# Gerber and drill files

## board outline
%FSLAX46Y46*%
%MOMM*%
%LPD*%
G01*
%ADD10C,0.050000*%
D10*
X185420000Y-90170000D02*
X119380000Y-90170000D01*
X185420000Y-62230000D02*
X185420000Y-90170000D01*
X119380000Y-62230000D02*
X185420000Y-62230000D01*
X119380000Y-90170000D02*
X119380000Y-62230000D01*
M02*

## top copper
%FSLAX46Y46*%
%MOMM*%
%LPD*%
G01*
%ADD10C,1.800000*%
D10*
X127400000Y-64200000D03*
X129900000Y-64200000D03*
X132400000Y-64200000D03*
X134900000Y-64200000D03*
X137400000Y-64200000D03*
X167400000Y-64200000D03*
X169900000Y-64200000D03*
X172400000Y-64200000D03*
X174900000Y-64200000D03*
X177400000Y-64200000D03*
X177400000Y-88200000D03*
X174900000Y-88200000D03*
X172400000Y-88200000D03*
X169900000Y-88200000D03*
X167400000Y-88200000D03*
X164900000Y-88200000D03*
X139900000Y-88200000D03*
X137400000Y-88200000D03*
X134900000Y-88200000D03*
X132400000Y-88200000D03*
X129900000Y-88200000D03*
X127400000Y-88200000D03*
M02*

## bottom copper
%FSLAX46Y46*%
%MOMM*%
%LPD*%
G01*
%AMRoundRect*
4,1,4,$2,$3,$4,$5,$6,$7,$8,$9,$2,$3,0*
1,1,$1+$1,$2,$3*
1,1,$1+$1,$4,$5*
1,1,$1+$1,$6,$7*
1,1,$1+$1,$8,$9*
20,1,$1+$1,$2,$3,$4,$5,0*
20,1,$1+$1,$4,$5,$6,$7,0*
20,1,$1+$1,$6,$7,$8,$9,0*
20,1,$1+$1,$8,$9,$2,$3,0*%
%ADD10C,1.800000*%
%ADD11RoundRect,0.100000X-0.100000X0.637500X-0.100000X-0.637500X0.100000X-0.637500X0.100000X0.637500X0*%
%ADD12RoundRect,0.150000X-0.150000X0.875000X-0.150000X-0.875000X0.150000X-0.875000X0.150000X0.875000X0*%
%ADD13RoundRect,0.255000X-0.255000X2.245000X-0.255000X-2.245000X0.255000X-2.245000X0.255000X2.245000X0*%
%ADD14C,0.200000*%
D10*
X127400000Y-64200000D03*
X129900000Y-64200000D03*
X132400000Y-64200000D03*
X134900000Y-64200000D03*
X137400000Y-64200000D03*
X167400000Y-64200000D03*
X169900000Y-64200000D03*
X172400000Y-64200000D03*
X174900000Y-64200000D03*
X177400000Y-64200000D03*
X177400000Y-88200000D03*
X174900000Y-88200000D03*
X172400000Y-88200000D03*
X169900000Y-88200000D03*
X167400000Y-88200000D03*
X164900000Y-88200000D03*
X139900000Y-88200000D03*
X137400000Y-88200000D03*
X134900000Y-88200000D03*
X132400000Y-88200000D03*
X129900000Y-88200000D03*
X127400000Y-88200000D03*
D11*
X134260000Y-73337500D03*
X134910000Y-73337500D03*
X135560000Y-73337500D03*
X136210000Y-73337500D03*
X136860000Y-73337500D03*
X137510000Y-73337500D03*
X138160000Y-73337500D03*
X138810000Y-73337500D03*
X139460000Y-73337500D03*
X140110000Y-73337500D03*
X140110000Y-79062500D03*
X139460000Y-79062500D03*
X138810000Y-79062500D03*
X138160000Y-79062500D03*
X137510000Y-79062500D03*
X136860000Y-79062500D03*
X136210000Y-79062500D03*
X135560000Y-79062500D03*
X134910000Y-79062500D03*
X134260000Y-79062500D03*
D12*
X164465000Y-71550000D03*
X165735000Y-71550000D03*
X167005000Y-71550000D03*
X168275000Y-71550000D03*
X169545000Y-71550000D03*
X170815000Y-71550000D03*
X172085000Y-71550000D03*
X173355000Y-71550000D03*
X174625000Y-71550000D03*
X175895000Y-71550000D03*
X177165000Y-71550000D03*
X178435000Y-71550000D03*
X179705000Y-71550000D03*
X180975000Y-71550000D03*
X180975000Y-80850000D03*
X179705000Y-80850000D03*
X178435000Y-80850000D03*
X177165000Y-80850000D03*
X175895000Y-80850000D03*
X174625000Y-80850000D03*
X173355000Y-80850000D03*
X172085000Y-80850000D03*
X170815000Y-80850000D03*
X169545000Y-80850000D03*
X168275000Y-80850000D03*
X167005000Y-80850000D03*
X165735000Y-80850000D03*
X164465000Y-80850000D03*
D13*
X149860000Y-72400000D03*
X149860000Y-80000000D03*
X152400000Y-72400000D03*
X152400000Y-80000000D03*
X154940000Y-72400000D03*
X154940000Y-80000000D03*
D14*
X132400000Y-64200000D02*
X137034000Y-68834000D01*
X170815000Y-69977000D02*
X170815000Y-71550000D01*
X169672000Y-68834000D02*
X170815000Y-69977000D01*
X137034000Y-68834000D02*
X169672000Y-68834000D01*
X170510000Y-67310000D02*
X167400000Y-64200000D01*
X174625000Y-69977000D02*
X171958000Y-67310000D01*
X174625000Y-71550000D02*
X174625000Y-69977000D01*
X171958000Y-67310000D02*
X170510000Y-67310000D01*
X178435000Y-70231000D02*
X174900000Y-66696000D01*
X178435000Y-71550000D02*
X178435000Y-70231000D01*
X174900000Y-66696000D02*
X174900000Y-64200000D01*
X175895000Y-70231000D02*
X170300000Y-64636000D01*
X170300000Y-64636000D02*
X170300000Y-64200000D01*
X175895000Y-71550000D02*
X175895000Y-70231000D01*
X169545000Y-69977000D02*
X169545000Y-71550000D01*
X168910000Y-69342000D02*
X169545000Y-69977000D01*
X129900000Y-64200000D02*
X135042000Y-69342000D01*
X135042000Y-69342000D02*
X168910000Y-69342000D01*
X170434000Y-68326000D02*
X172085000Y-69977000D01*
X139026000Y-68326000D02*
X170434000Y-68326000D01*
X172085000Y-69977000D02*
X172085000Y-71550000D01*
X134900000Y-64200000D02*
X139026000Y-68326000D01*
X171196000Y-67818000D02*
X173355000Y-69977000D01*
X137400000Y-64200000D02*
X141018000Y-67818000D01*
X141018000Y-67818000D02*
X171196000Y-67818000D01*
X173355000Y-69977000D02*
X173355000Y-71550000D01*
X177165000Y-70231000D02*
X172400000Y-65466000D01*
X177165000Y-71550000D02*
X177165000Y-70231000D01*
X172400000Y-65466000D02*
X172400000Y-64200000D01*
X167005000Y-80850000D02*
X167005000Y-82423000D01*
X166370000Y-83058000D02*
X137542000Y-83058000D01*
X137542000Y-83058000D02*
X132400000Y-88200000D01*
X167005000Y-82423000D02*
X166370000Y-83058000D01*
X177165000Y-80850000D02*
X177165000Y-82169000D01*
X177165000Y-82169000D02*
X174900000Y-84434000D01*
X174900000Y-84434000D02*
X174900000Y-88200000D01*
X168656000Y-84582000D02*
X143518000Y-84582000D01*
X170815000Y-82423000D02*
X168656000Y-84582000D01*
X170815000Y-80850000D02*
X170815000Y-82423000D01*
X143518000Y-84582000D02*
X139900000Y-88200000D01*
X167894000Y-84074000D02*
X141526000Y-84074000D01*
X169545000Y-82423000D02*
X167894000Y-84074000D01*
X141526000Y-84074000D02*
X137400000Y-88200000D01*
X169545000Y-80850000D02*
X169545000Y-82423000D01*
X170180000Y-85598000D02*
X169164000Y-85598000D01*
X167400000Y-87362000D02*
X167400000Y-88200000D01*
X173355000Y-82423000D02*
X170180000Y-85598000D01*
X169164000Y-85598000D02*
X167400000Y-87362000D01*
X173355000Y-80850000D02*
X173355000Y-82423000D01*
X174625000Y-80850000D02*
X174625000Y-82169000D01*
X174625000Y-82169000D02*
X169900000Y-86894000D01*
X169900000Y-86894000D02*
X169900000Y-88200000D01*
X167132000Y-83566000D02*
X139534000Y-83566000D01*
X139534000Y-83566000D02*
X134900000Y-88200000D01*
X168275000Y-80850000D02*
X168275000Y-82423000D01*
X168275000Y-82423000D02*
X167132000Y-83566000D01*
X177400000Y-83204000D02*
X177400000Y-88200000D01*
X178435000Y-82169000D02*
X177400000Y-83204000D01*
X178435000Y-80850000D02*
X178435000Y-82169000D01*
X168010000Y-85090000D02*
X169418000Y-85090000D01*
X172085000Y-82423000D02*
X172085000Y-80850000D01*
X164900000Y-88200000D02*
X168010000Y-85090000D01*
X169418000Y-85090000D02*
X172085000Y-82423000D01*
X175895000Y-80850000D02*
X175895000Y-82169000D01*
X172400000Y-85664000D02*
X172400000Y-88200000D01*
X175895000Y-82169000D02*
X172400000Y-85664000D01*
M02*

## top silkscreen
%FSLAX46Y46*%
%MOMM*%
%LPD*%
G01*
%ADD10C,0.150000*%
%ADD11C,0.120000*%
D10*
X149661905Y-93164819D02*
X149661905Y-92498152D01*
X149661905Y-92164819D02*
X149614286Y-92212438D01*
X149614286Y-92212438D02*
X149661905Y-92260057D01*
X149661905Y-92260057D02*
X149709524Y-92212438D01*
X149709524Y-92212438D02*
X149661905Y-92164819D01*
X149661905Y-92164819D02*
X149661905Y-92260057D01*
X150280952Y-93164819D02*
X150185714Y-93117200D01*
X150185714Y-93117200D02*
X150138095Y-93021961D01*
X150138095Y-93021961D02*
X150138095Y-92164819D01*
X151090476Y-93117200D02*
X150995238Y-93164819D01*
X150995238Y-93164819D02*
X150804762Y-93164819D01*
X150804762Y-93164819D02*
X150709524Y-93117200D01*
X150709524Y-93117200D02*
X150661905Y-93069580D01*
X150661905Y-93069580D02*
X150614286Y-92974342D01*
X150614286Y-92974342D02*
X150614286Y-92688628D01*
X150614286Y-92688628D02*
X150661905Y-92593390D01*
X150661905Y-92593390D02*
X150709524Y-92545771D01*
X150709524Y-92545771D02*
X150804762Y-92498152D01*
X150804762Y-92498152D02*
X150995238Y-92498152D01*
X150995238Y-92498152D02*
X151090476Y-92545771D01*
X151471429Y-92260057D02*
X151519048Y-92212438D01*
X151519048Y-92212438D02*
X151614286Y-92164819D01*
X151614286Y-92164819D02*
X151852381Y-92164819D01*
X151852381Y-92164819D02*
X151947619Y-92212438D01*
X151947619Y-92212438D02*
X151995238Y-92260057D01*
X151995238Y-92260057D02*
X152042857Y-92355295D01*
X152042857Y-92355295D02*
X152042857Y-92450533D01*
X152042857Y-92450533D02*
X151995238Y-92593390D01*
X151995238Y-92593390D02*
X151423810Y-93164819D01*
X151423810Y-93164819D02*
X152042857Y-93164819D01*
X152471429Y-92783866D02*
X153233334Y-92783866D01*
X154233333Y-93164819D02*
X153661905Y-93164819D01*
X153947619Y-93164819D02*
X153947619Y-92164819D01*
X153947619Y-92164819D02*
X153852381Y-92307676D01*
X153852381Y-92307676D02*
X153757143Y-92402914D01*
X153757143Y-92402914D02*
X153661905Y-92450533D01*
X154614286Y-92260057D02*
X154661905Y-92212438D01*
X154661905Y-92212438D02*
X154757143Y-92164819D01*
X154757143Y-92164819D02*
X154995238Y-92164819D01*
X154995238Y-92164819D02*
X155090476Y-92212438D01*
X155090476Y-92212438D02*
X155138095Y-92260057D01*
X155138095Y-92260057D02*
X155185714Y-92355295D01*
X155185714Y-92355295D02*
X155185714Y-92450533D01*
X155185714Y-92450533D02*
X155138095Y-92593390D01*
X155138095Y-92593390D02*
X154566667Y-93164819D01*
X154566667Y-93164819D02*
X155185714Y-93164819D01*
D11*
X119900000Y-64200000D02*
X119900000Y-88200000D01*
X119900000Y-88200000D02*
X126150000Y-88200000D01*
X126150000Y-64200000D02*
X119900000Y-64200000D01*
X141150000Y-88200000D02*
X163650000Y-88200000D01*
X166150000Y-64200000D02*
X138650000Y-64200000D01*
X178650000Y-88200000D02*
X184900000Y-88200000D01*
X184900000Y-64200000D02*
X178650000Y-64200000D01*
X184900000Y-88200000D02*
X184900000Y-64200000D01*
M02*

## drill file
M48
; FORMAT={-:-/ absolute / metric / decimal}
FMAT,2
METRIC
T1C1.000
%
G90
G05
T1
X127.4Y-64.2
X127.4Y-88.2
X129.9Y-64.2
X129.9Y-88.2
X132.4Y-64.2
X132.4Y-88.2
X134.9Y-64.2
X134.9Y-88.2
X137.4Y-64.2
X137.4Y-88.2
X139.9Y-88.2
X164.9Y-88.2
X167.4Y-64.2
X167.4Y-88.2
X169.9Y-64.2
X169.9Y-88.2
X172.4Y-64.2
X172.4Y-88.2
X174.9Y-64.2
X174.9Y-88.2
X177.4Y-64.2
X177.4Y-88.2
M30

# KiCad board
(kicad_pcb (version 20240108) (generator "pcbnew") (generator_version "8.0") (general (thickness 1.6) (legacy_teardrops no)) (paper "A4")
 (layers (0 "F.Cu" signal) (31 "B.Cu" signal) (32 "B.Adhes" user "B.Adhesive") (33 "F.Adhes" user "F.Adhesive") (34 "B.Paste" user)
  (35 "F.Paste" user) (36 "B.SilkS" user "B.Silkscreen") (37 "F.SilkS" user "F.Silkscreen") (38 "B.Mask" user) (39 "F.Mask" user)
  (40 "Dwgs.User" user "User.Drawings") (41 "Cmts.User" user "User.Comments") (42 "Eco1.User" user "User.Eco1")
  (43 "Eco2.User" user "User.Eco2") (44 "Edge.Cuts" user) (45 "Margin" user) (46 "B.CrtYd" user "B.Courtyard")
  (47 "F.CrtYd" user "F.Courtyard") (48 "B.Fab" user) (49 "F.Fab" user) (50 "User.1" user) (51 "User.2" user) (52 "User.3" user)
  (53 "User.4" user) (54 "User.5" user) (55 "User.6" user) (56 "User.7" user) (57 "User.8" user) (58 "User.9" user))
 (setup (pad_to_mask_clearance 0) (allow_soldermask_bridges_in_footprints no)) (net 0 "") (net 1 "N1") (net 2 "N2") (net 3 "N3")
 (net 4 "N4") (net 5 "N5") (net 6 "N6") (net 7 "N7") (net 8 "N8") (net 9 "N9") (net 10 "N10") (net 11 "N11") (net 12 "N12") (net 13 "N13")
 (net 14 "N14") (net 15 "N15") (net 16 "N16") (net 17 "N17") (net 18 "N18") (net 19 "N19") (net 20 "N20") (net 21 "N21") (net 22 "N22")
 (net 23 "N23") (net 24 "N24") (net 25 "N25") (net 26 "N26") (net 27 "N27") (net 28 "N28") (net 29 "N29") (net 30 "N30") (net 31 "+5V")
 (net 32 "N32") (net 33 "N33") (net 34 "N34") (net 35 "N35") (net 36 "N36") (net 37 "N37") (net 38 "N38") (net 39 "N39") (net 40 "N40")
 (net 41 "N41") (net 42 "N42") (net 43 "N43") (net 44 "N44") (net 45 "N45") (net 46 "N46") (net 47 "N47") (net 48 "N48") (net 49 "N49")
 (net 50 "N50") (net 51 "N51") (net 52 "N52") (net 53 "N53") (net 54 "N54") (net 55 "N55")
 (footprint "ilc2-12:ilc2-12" (layer "F.Cu") (at 152.4 76.2)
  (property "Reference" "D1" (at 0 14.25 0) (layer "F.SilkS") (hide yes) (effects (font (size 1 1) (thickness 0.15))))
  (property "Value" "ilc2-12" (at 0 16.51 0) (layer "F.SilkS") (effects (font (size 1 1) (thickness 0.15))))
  (fp_line (start -32.5 -12) (end -32.5 12) (stroke (width 0.12) (type solid)) (layer "F.SilkS"))
  (fp_line (start -32.5 12) (end -26.25 12) (stroke (width 0.12) (type solid)) (layer "F.SilkS"))
  (fp_line (start -26.25 -12) (end -32.5 -12) (stroke (width 0.12) (type solid)) (layer "F.SilkS"))
  (fp_line (start -11.25 12) (end 11.25 12) (stroke (width 0.12) (type solid)) (layer "F.SilkS"))
  (fp_line (start 13.75 -12) (end -13.75 -12) (stroke (width 0.12) (type solid)) (layer "F.SilkS"))
  (fp_line (start 26.25 12) (end 32.5 12) (stroke (width 0.12) (type solid)) (layer "F.SilkS"))
  (fp_line (start 32.5 -12) (end 26.25 -12) (stroke (width 0.12) (type solid)) (layer "F.SilkS"))
  (fp_line (start 32.5 12) (end 32.5 -12) (stroke (width 0.12) (type solid)) (layer "F.SilkS"))
  (pad "1" thru_hole circle (at -25 -12) (size 1.8 1.8) (drill 1) (layers "*.Cu" "*.Mask") (remove_unused_layers no) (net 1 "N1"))
  (pad "2" thru_hole circle (at -22.5 -12) (size 1.8 1.8) (drill 1) (layers "*.Cu" "*.Mask") (remove_unused_layers no) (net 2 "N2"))
  (pad "3" thru_hole circle (at -20 -12) (size 1.8 1.8) (drill 1) (layers "*.Cu" "*.Mask") (remove_unused_layers no) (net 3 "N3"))
  (pad "4" thru_hole circle (at -17.5 -12) (size 1.8 1.8) (drill 1) (layers "*.Cu" "*.Mask") (remove_unused_layers no) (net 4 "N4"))
  (pad "5" thru_hole circle (at -15 -12) (size 1.8 1.8) (drill 1) (layers "*.Cu" "*.Mask") (remove_unused_layers no) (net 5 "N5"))
  (pad "6" thru_hole circle (at 15 -12) (size 1.8 1.8) (drill 1) (layers "*.Cu" "*.Mask") (remove_unused_layers no) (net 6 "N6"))
  (pad "7" thru_hole circle (at 17.5 -12) (size 1.8 1.8) (drill 1) (layers "*.Cu" "*.Mask") (remove_unused_layers no) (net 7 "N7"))
  (pad "8" thru_hole circle (at 20 -12) (size 1.8 1.8) (drill 1) (layers "*.Cu" "*.Mask") (remove_unused_layers no) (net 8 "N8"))
  (pad "9" thru_hole circle (at 22.5 -12) (size 1.8 1.8) (drill 1) (layers "*.Cu" "*.Mask") (remove_unused_layers no) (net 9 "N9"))
  (pad "10" thru_hole circle (at 25 -12) (size 1.8 1.8) (drill 1) (layers "*.Cu" "*.Mask") (remove_unused_layers no) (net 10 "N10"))
  (pad "11" thru_hole circle (at 25 12) (size 1.8 1.8) (drill 1) (layers "*.Cu" "*.Mask") (remove_unused_layers no) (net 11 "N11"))
  (pad "12" thru_hole circle (at 22.5 12) (size 1.8 1.8) (drill 1) (layers "*.Cu" "*.Mask") (remove_unused_layers no) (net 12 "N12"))
  (pad "13" thru_hole circle (at 20 12) (size 1.8 1.8) (drill 1) (layers "*.Cu" "*.Mask") (remove_unused_layers no) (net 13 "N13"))
  (pad "14" thru_hole circle (at 17.5 12) (size 1.8 1.8) (drill 1) (layers "*.Cu" "*.Mask") (remove_unused_layers no) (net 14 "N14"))
  (pad "15" thru_hole circle (at 15 12) (size 1.8 1.8) (drill 1) (layers "*.Cu" "*.Mask") (remove_unused_layers no) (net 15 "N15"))
  (pad "16" thru_hole circle (at 12.5 12) (size 1.8 1.8) (drill 1) (layers "*.Cu" "*.Mask") (remove_unused_layers no) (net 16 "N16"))
  (pad "17" thru_hole circle (at -12.5 12) (size 1.8 1.8) (drill 1) (layers "*.Cu" "*.Mask") (remove_unused_layers no) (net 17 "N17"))
  (pad "18" thru_hole circle (at -15 12) (size 1.8 1.8) (drill 1) (layers "*.Cu" "*.Mask") (remove_unused_layers no) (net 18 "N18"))
  (pad "19" thru_hole circle (at -17.5 12) (size 1.8 1.8) (drill 1) (layers "*.Cu" "*.Mask") (remove_unused_layers no) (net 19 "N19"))
  (pad "20" thru_hole circle (at -20 12) (size 1.8 1.8) (drill 1) (layers "*.Cu" "*.Mask") (remove_unused_layers no) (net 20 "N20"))
  (pad "21" thru_hole circle (at -22.5 12) (size 1.8 1.8) (drill 1) (layers "*.Cu" "*.Mask") (remove_unused_layers no) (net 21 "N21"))
  (pad "22" thru_hole circle (at -25 12) (size 1.8 1.8) (drill 1) (layers "*.Cu" "*.Mask") (remove_unused_layers no) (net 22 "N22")))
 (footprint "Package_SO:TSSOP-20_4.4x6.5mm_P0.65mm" (layer "B.Cu") (at 137.185 76.2 -90)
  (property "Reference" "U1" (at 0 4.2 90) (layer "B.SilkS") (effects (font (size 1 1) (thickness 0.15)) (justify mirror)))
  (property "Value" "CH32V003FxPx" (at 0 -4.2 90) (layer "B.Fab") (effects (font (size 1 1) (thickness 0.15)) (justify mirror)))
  (pad "1" smd roundrect (at -2.8625 2.925 270) (size 1.475 0.4) (layers "B.Cu" "B.Paste" "B.Mask") (roundrect_rratio 0.25) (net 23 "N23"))
  (pad "2" smd roundrect (at -2.8625 2.275 270) (size 1.475 0.4) (layers "B.Cu" "B.Paste" "B.Mask") (roundrect_rratio 0.25) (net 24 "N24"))
  (pad "3" smd roundrect (at -2.8625 1.625 270) (size 1.475 0.4) (layers "B.Cu" "B.Paste" "B.Mask") (roundrect_rratio 0.25) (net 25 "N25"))
  (pad "4" smd roundrect (at -2.8625 0.975 270) (size 1.475 0.4) (layers "B.Cu" "B.Paste" "B.Mask") (roundrect_rratio 0.25) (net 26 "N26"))
  (pad "5" smd roundrect (at -2.8625 0.325 270) (size 1.475 0.4) (layers "B.Cu" "B.Paste" "B.Mask") (roundrect_rratio 0.25) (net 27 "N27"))
  (pad "6" smd roundrect (at -2.8625 -0.325 270) (size 1.475 0.4) (layers "B.Cu" "B.Paste" "B.Mask") (roundrect_rratio 0.25) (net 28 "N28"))
  (pad "7" smd roundrect (at -2.8625 -0.975 270) (size 1.475 0.4) (layers "B.Cu" "B.Paste" "B.Mask") (roundrect_rratio 0.25) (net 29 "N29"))
  (pad "8" smd roundrect (at -2.8625 -1.625 270) (size 1.475 0.4) (layers "B.Cu" "B.Paste" "B.Mask") (roundrect_rratio 0.25) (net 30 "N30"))
  (pad "9" smd roundrect (at -2.8625 -2.275 270) (size 1.475 0.4) (layers "B.Cu" "B.Paste" "B.Mask") (roundrect_rratio 0.25) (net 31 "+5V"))
  (pad "10" smd roundrect (at -2.8625 -2.925 270) (size 1.475 0.4) (layers "B.Cu" "B.Paste" "B.Mask") (roundrect_rratio 0.25) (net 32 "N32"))
  (pad "11" smd roundrect (at 2.8625 -2.925 270) (size 1.475 0.4) (layers "B.Cu" "B.Paste" "B.Mask") (roundrect_rratio 0.25) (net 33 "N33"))
  (pad "12" smd roundrect (at 2.8625 -2.275 270) (size 1.475 0.4) (layers "B.Cu" "B.Paste" "B.Mask") (roundrect_rratio 0.25) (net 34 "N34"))
  (pad "13" smd roundrect (at 2.8625 -1.625 270) (size 1.475 0.4) (layers "B.Cu" "B.Paste" "B.Mask") (roundrect_rratio 0.25) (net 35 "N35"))
  (pad "14" smd roundrect (at 2.8625 -0.975 270) (size 1.475 0.4) (layers "B.Cu" "B.Paste" "B.Mask") (roundrect_rratio 0.25) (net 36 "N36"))
  (pad "15" smd roundrect (at 2.8625 -0.325 270) (size 1.475 0.4) (layers "B.Cu" "B.Paste" "B.Mask") (roundrect_rratio 0.25) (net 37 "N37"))
  (pad "16" smd roundrect (at 2.8625 0.325 270) (size 1.475 0.4) (layers "B.Cu" "B.Paste" "B.Mask") (roundrect_rratio 0.25) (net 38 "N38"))
  (pad "17" smd roundrect (at 2.8625 0.975 270) (size 1.475 0.4) (layers "B.Cu" "B.Paste" "B.Mask") (roundrect_rratio 0.25) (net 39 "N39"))
  (pad "18" smd roundrect (at 2.8625 1.625 270) (size 1.475 0.4) (layers "B.Cu" "B.Paste" "B.Mask") (roundrect_rratio 0.25) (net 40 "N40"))
  (pad "19" smd roundrect (at 2.8625 2.275 270) (size 1.475 0.4) (layers "B.Cu" "B.Paste" "B.Mask") (roundrect_rratio 0.25) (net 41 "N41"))
  (pad "20" smd roundrect (at 2.8625 2.925 270) (size 1.475 0.4) (layers "B.Cu" "B.Paste" "B.Mask") (roundrect_rratio 0.25) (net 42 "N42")))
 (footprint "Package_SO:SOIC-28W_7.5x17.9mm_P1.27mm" (layer "B.Cu") (at 172.72 76.2 -90)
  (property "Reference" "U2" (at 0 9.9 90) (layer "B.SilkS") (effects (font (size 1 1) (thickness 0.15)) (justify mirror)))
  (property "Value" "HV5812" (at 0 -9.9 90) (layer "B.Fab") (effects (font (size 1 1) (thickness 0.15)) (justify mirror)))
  (pad "1" smd roundrect (at -4.65 8.255 270) (size 2.05 0.6) (layers "B.Cu" "B.Paste" "B.Mask") (roundrect_rratio 0.25) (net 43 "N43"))
  (pad "2" smd roundrect (at -4.65 6.985 270) (size 2.05 0.6) (layers "B.Cu" "B.Paste" "B.Mask") (roundrect_rratio 0.25) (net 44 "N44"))
  (pad "3" smd roundrect (at -4.65 5.715 270) (size 2.05 0.6) (layers "B.Cu" "B.Paste" "B.Mask") (roundrect_rratio 0.25) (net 22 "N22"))
  (pad "4" smd roundrect (at -4.65 4.445 270) (size 2.05 0.6) (layers "B.Cu" "B.Paste" "B.Mask") (roundrect_rratio 0.25) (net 21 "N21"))
  (pad "5" smd roundrect (at -4.65 3.175 270) (size 2.05 0.6) (layers "B.Cu" "B.Paste" "B.Mask") (roundrect_rratio 0.25) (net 2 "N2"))
  (pad "6" smd roundrect (at -4.65 1.905 270) (size 2.05 0.6) (layers "B.Cu" "B.Paste" "B.Mask") (roundrect_rratio 0.25) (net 3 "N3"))
  (pad "7" smd roundrect (at -4.65 0.635 270) (size 2.05 0.6) (layers "B.Cu" "B.Paste" "B.Mask") (roundrect_rratio 0.25) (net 4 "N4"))
  (pad "8" smd roundrect (at -4.65 -0.635 270) (size 2.05 0.6) (layers "B.Cu" "B.Paste" "B.Mask") (roundrect_rratio 0.25) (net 5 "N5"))
  (pad "9" smd roundrect (at -4.65 -1.905 270) (size 2.05 0.6) (layers "B.Cu" "B.Paste" "B.Mask") (roundrect_rratio 0.25) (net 6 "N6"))
  (pad "10" smd roundrect (at -4.65 -3.175 270) (size 2.05 0.6) (layers "B.Cu" "B.Paste" "B.Mask") (roundrect_rratio 0.25) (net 7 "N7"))
  (pad "11" smd roundrect (at -4.65 -4.445 270) (size 2.05 0.6) (layers "B.Cu" "B.Paste" "B.Mask") (roundrect_rratio 0.25) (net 8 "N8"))
  (pad "12" smd roundrect (at -4.65 -5.715 270) (size 2.05 0.6) (layers "B.Cu" "B.Paste" "B.Mask") (roundrect_rratio 0.25) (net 9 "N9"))
  (pad "13" smd roundrect (at -4.65 -6.985 270) (size 2.05 0.6) (layers "B.Cu" "B.Paste" "B.Mask") (roundrect_rratio 0.25) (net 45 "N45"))
  (pad "14" smd roundrect (at -4.65 -8.255 270) (size 2.05 0.6) (layers "B.Cu" "B.Paste" "B.Mask") (roundrect_rratio 0.25) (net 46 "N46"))
  (pad "15" smd roundrect (at 4.65 -8.255 270) (size 2.05 0.6) (layers "B.Cu" "B.Paste" "B.Mask") (roundrect_rratio 0.25) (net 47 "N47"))
  (pad "16" smd roundrect (at 4.65 -6.985 270) (size 2.05 0.6) (layers "B.Cu" "B.Paste" "B.Mask") (roundrect_rratio 0.25) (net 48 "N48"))
  (pad "17" smd roundrect (at 4.65 -5.715 270) (size 2.05 0.6) (layers "B.Cu" "B.Paste" "B.Mask") (roundrect_rratio 0.25) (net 11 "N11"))
  (pad "18" smd roundrect (at 4.65 -4.445 270) (size 2.05 0.6) (layers "B.Cu" "B.Paste" "B.Mask") (roundrect_rratio 0.25) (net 12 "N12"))
  (pad "19" smd roundrect (at 4.65 -3.175 270) (size 2.05 0.6) (layers "B.Cu" "B.Paste" "B.Mask") (roundrect_rratio 0.25) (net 13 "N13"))
  (pad "20" smd roundrect (at 4.65 -1.905 270) (size 2.05 0.6) (layers "B.Cu" "B.Paste" "B.Mask") (roundrect_rratio 0.25) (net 14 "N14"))
  (pad "21" smd roundrect (at 4.65 -0.635 270) (size 2.05 0.6) (layers "B.Cu" "B.Paste" "B.Mask") (roundrect_rratio 0.25) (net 15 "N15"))
  (pad "22" smd roundrect (at 4.65 0.635 270) (size 2.05 0.6) (layers "B.Cu" "B.Paste" "B.Mask") (roundrect_rratio 0.25) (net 16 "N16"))
  (pad "23" smd roundrect (at 4.65 1.905 270) (size 2.05 0.6) (layers "B.Cu" "B.Paste" "B.Mask") (roundrect_rratio 0.25) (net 17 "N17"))
  (pad "24" smd roundrect (at 4.65 3.175 270) (size 2.05 0.6) (layers "B.Cu" "B.Paste" "B.Mask") (roundrect_rratio 0.25) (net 18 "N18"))
  (pad "25" smd roundrect (at 4.65 4.445 270) (size 2.05 0.6) (layers "B.Cu" "B.Paste" "B.Mask") (roundrect_rratio 0.25) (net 19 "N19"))
  (pad "26" smd roundrect (at 4.65 5.715 270) (size 2.05 0.6) (layers "B.Cu" "B.Paste" "B.Mask") (roundrect_rratio 0.25) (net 20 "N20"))
  (pad "27" smd roundrect (at 4.65 6.985 270) (size 2.05 0.6) (layers "B.Cu" "B.Paste" "B.Mask") (roundrect_rratio 0.25) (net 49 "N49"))
  (pad "28" smd roundrect (at 4.65 8.255 270) (size 2.05 0.6) (layers "B.Cu" "B.Paste" "B.Mask") (roundrect_rratio 0.25) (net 31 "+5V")))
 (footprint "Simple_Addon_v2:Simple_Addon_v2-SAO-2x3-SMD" (layer "B.Cu") (at 152.4 76.2 -90)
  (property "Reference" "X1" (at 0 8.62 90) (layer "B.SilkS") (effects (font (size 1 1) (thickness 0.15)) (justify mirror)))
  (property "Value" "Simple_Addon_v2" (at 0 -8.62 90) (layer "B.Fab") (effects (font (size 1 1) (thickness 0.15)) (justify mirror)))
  (pad "1" smd roundrect (at -3.8 2.54 270) (size 5 1.02) (layers "B.Cu" "B.Paste" "B.Mask") (roundrect_rratio 0.25) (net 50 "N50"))
  (pad "2" smd roundrect (at 3.8 2.54 270) (size 5 1.02) (layers "B.Cu" "B.Paste" "B.Mask") (roundrect_rratio 0.25) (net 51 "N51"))
  (pad "3" smd roundrect (at -3.8 0 270) (size 5 1.02) (layers "B.Cu" "B.Paste" "B.Mask") (roundrect_rratio 0.25) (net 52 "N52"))
  (pad "4" smd roundrect (at 3.8 0 270) (size 5 1.02) (layers "B.Cu" "B.Paste" "B.Mask") (roundrect_rratio 0.25) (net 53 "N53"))
  (pad "5" smd roundrect (at -3.8 -2.54 270) (size 5 1.02) (layers "B.Cu" "B.Paste" "B.Mask") (roundrect_rratio 0.25) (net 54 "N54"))
  (pad "6" smd roundrect (at 3.8 -2.54 270) (size 5 1.02) (layers "B.Cu" "B.Paste" "B.Mask") (roundrect_rratio 0.25) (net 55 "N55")))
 (gr_line (start 185.42 90.17) (end 119.38 90.17) (stroke (width 0.05) (type default)) (layer "Edge.Cuts"))
 (gr_line (start 185.42 62.23) (end 185.42 90.17) (stroke (width 0.05) (type default)) (layer "Edge.Cuts"))
 (gr_line (start 119.38 62.23) (end 185.42 62.23) (stroke (width 0.05) (type default)) (layer "Edge.Cuts"))
 (gr_line (start 119.38 90.17) (end 119.38 62.23) (stroke (width 0.05) (type default)) (layer "Edge.Cuts"))
 (segment (start 132.4 64.2) (end 137.034 68.834) (width 0.2) (layer "B.Cu") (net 3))
 (segment (start 170.815 69.977) (end 170.815 71.55) (width 0.2) (layer "B.Cu") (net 3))
 (segment (start 169.672 68.834) (end 170.815 69.977) (width 0.2) (layer "B.Cu") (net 3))
 (segment (start 137.034 68.834) (end 169.672 68.834) (width 0.2) (layer "B.Cu") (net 3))
 (segment (start 170.51 67.31) (end 167.4 64.2) (width 0.2) (layer "B.Cu") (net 6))
 (segment (start 174.625 69.977) (end 171.958 67.31) (width 0.2) (layer "B.Cu") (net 6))
 (segment (start 174.625 71.55) (end 174.625 69.977) (width 0.2) (layer "B.Cu") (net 6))
 (segment (start 171.958 67.31) (end 170.51 67.31) (width 0.2) (layer "B.Cu") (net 6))
 (segment (start 178.435 70.231) (end 174.9 66.696) (width 0.2) (layer "B.Cu") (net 9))
 (segment (start 178.435 71.55) (end 178.435 70.231) (width 0.2) (layer "B.Cu") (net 9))
 (segment (start 174.9 66.696) (end 174.9 64.2) (width 0.2) (layer "B.Cu") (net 9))
 (segment (start 175.895 70.231) (end 170.3 64.636) (width 0.2) (layer "B.Cu") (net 7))
 (segment (start 170.3 64.636) (end 170.3 64.2) (width 0.2) (layer "B.Cu") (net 7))
 (segment (start 175.895 71.55) (end 175.895 70.231) (width 0.2) (layer "B.Cu") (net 7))
 (segment (start 169.545 69.977) (end 169.545 71.55) (width 0.2) (layer "B.Cu") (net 2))
 (segment (start 168.91 69.342) (end 169.545 69.977) (width 0.2) (layer "B.Cu") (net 2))
 (segment (start 129.9 64.2) (end 135.042 69.342) (width 0.2) (layer "B.Cu") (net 2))
 (segment (start 135.042 69.342) (end 168.91 69.342) (width 0.2) (layer "B.Cu") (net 2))
 (segment (start 170.434 68.326) (end 172.085 69.977) (width 0.2) (layer "B.Cu") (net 4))
 (segment (start 139.026 68.326) (end 170.434 68.326) (width 0.2) (layer "B.Cu") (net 4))
 (segment (start 172.085 69.977) (end 172.085 71.55) (width 0.2) (layer "B.Cu") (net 4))
 (segment (start 134.9 64.2) (end 139.026 68.326) (width 0.2) (layer "B.Cu") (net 4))
 (segment (start 171.196 67.818) (end 173.355 69.977) (width 0.2) (layer "B.Cu") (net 5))
 (segment (start 137.4 64.2) (end 141.018 67.818) (width 0.2) (layer "B.Cu") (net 5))
 (segment (start 141.018 67.818) (end 171.196 67.818) (width 0.2) (layer "B.Cu") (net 5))
 (segment (start 173.355 69.977) (end 173.355 71.55) (width 0.2) (layer "B.Cu") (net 5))
 (segment (start 177.165 70.231) (end 172.4 65.466) (width 0.2) (layer "B.Cu") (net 8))
 (segment (start 177.165 71.55) (end 177.165 70.231) (width 0.2) (layer "B.Cu") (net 8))
 (segment (start 172.4 65.466) (end 172.4 64.2) (width 0.2) (layer "B.Cu") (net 8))
 (segment (start 167.005 80.85) (end 167.005 82.423) (width 0.2) (layer "B.Cu") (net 20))
 (segment (start 166.37 83.058) (end 137.542 83.058) (width 0.2) (layer "B.Cu") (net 20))
 (segment (start 137.542 83.058) (end 132.4 88.2) (width 0.2) (layer "B.Cu") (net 20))
 (segment (start 167.005 82.423) (end 166.37 83.058) (width 0.2) (layer "B.Cu") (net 20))
 (segment (start 177.165 80.85) (end 177.165 82.169) (width 0.2) (layer "B.Cu") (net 12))
 (segment (start 177.165 82.169) (end 174.9 84.434) (width 0.2) (layer "B.Cu") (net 12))
 (segment (start 174.9 84.434) (end 174.9 88.2) (width 0.2) (layer "B.Cu") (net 12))
 (segment (start 168.656 84.582) (end 143.518 84.582) (width 0.2) (layer "B.Cu") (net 17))
 (segment (start 170.815 82.423) (end 168.656 84.582) (width 0.2) (layer "B.Cu") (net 17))
 (segment (start 170.815 80.85) (end 170.815 82.423) (width 0.2) (layer "B.Cu") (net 17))
 (segment (start 143.518 84.582) (end 139.9 88.2) (width 0.2) (layer "B.Cu") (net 17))
 (segment (start 167.894 84.074) (end 141.526 84.074) (width 0.2) (layer "B.Cu") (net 18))
 (segment (start 169.545 82.423) (end 167.894 84.074) (width 0.2) (layer "B.Cu") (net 18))
 (segment (start 141.526 84.074) (end 137.4 88.2) (width 0.2) (layer "B.Cu") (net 18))
 (segment (start 169.545 80.85) (end 169.545 82.423) (width 0.2) (layer "B.Cu") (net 18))
 (segment (start 170.18 85.598) (end 169.164 85.598) (width 0.2) (layer "B.Cu") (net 15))
 (segment (start 167.4 87.362) (end 167.4 88.2) (width 0.2) (layer "B.Cu") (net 15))
 (segment (start 173.355 82.423) (end 170.18 85.598) (width 0.2) (layer "B.Cu") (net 15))
 (segment (start 169.164 85.598) (end 167.4 87.362) (width 0.2) (layer "B.Cu") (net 15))
 (segment (start 173.355 80.85) (end 173.355 82.423) (width 0.2) (layer "B.Cu") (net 15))
 (segment (start 174.625 80.85) (end 174.625 82.169) (width 0.2) (layer "B.Cu") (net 14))
 (segment (start 174.625 82.169) (end 169.9 86.894) (width 0.2) (layer "B.Cu") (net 14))
 (segment (start 169.9 86.894) (end 169.9 88.2) (width 0.2) (layer "B.Cu") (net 14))
 (segment (start 167.132 83.566) (end 139.534 83.566) (width 0.2) (layer "B.Cu") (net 19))
 (segment (start 139.534 83.566) (end 134.9 88.2) (width 0.2) (layer "B.Cu") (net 19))
 (segment (start 168.275 80.85) (end 168.275 82.423) (width 0.2) (layer "B.Cu") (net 19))
 (segment (start 168.275 82.423) (end 167.132 83.566) (width 0.2) (layer "B.Cu") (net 19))
 (segment (start 177.4 83.204) (end 177.4 88.2) (width 0.2) (layer "B.Cu") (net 11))
 (segment (start 178.435 82.169) (end 177.4 83.204) (width 0.2) (layer "B.Cu") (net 11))
 (segment (start 178.435 80.85) (end 178.435 82.169) (width 0.2) (layer "B.Cu") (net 11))
 (segment (start 168.01 85.09) (end 169.418 85.09) (width 0.2) (layer "B.Cu") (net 16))
 (segment (start 172.085 82.423) (end 172.085 80.85) (width 0.2) (layer "B.Cu") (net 16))
 (segment (start 164.9 88.2) (end 168.01 85.09) (width 0.2) (layer "B.Cu") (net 16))
 (segment (start 169.418 85.09) (end 172.085 82.423) (width 0.2) (layer "B.Cu") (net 16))
 (segment (start 175.895 80.85) (end 175.895 82.169) (width 0.2) (layer "B.Cu") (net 13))
 (segment (start 172.4 85.664) (end 172.4 88.2) (width 0.2) (layer "B.Cu") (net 13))
 (segment (start 175.895 82.169) (end 172.4 85.664) (width 0.2) (layer "B.Cu") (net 13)))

